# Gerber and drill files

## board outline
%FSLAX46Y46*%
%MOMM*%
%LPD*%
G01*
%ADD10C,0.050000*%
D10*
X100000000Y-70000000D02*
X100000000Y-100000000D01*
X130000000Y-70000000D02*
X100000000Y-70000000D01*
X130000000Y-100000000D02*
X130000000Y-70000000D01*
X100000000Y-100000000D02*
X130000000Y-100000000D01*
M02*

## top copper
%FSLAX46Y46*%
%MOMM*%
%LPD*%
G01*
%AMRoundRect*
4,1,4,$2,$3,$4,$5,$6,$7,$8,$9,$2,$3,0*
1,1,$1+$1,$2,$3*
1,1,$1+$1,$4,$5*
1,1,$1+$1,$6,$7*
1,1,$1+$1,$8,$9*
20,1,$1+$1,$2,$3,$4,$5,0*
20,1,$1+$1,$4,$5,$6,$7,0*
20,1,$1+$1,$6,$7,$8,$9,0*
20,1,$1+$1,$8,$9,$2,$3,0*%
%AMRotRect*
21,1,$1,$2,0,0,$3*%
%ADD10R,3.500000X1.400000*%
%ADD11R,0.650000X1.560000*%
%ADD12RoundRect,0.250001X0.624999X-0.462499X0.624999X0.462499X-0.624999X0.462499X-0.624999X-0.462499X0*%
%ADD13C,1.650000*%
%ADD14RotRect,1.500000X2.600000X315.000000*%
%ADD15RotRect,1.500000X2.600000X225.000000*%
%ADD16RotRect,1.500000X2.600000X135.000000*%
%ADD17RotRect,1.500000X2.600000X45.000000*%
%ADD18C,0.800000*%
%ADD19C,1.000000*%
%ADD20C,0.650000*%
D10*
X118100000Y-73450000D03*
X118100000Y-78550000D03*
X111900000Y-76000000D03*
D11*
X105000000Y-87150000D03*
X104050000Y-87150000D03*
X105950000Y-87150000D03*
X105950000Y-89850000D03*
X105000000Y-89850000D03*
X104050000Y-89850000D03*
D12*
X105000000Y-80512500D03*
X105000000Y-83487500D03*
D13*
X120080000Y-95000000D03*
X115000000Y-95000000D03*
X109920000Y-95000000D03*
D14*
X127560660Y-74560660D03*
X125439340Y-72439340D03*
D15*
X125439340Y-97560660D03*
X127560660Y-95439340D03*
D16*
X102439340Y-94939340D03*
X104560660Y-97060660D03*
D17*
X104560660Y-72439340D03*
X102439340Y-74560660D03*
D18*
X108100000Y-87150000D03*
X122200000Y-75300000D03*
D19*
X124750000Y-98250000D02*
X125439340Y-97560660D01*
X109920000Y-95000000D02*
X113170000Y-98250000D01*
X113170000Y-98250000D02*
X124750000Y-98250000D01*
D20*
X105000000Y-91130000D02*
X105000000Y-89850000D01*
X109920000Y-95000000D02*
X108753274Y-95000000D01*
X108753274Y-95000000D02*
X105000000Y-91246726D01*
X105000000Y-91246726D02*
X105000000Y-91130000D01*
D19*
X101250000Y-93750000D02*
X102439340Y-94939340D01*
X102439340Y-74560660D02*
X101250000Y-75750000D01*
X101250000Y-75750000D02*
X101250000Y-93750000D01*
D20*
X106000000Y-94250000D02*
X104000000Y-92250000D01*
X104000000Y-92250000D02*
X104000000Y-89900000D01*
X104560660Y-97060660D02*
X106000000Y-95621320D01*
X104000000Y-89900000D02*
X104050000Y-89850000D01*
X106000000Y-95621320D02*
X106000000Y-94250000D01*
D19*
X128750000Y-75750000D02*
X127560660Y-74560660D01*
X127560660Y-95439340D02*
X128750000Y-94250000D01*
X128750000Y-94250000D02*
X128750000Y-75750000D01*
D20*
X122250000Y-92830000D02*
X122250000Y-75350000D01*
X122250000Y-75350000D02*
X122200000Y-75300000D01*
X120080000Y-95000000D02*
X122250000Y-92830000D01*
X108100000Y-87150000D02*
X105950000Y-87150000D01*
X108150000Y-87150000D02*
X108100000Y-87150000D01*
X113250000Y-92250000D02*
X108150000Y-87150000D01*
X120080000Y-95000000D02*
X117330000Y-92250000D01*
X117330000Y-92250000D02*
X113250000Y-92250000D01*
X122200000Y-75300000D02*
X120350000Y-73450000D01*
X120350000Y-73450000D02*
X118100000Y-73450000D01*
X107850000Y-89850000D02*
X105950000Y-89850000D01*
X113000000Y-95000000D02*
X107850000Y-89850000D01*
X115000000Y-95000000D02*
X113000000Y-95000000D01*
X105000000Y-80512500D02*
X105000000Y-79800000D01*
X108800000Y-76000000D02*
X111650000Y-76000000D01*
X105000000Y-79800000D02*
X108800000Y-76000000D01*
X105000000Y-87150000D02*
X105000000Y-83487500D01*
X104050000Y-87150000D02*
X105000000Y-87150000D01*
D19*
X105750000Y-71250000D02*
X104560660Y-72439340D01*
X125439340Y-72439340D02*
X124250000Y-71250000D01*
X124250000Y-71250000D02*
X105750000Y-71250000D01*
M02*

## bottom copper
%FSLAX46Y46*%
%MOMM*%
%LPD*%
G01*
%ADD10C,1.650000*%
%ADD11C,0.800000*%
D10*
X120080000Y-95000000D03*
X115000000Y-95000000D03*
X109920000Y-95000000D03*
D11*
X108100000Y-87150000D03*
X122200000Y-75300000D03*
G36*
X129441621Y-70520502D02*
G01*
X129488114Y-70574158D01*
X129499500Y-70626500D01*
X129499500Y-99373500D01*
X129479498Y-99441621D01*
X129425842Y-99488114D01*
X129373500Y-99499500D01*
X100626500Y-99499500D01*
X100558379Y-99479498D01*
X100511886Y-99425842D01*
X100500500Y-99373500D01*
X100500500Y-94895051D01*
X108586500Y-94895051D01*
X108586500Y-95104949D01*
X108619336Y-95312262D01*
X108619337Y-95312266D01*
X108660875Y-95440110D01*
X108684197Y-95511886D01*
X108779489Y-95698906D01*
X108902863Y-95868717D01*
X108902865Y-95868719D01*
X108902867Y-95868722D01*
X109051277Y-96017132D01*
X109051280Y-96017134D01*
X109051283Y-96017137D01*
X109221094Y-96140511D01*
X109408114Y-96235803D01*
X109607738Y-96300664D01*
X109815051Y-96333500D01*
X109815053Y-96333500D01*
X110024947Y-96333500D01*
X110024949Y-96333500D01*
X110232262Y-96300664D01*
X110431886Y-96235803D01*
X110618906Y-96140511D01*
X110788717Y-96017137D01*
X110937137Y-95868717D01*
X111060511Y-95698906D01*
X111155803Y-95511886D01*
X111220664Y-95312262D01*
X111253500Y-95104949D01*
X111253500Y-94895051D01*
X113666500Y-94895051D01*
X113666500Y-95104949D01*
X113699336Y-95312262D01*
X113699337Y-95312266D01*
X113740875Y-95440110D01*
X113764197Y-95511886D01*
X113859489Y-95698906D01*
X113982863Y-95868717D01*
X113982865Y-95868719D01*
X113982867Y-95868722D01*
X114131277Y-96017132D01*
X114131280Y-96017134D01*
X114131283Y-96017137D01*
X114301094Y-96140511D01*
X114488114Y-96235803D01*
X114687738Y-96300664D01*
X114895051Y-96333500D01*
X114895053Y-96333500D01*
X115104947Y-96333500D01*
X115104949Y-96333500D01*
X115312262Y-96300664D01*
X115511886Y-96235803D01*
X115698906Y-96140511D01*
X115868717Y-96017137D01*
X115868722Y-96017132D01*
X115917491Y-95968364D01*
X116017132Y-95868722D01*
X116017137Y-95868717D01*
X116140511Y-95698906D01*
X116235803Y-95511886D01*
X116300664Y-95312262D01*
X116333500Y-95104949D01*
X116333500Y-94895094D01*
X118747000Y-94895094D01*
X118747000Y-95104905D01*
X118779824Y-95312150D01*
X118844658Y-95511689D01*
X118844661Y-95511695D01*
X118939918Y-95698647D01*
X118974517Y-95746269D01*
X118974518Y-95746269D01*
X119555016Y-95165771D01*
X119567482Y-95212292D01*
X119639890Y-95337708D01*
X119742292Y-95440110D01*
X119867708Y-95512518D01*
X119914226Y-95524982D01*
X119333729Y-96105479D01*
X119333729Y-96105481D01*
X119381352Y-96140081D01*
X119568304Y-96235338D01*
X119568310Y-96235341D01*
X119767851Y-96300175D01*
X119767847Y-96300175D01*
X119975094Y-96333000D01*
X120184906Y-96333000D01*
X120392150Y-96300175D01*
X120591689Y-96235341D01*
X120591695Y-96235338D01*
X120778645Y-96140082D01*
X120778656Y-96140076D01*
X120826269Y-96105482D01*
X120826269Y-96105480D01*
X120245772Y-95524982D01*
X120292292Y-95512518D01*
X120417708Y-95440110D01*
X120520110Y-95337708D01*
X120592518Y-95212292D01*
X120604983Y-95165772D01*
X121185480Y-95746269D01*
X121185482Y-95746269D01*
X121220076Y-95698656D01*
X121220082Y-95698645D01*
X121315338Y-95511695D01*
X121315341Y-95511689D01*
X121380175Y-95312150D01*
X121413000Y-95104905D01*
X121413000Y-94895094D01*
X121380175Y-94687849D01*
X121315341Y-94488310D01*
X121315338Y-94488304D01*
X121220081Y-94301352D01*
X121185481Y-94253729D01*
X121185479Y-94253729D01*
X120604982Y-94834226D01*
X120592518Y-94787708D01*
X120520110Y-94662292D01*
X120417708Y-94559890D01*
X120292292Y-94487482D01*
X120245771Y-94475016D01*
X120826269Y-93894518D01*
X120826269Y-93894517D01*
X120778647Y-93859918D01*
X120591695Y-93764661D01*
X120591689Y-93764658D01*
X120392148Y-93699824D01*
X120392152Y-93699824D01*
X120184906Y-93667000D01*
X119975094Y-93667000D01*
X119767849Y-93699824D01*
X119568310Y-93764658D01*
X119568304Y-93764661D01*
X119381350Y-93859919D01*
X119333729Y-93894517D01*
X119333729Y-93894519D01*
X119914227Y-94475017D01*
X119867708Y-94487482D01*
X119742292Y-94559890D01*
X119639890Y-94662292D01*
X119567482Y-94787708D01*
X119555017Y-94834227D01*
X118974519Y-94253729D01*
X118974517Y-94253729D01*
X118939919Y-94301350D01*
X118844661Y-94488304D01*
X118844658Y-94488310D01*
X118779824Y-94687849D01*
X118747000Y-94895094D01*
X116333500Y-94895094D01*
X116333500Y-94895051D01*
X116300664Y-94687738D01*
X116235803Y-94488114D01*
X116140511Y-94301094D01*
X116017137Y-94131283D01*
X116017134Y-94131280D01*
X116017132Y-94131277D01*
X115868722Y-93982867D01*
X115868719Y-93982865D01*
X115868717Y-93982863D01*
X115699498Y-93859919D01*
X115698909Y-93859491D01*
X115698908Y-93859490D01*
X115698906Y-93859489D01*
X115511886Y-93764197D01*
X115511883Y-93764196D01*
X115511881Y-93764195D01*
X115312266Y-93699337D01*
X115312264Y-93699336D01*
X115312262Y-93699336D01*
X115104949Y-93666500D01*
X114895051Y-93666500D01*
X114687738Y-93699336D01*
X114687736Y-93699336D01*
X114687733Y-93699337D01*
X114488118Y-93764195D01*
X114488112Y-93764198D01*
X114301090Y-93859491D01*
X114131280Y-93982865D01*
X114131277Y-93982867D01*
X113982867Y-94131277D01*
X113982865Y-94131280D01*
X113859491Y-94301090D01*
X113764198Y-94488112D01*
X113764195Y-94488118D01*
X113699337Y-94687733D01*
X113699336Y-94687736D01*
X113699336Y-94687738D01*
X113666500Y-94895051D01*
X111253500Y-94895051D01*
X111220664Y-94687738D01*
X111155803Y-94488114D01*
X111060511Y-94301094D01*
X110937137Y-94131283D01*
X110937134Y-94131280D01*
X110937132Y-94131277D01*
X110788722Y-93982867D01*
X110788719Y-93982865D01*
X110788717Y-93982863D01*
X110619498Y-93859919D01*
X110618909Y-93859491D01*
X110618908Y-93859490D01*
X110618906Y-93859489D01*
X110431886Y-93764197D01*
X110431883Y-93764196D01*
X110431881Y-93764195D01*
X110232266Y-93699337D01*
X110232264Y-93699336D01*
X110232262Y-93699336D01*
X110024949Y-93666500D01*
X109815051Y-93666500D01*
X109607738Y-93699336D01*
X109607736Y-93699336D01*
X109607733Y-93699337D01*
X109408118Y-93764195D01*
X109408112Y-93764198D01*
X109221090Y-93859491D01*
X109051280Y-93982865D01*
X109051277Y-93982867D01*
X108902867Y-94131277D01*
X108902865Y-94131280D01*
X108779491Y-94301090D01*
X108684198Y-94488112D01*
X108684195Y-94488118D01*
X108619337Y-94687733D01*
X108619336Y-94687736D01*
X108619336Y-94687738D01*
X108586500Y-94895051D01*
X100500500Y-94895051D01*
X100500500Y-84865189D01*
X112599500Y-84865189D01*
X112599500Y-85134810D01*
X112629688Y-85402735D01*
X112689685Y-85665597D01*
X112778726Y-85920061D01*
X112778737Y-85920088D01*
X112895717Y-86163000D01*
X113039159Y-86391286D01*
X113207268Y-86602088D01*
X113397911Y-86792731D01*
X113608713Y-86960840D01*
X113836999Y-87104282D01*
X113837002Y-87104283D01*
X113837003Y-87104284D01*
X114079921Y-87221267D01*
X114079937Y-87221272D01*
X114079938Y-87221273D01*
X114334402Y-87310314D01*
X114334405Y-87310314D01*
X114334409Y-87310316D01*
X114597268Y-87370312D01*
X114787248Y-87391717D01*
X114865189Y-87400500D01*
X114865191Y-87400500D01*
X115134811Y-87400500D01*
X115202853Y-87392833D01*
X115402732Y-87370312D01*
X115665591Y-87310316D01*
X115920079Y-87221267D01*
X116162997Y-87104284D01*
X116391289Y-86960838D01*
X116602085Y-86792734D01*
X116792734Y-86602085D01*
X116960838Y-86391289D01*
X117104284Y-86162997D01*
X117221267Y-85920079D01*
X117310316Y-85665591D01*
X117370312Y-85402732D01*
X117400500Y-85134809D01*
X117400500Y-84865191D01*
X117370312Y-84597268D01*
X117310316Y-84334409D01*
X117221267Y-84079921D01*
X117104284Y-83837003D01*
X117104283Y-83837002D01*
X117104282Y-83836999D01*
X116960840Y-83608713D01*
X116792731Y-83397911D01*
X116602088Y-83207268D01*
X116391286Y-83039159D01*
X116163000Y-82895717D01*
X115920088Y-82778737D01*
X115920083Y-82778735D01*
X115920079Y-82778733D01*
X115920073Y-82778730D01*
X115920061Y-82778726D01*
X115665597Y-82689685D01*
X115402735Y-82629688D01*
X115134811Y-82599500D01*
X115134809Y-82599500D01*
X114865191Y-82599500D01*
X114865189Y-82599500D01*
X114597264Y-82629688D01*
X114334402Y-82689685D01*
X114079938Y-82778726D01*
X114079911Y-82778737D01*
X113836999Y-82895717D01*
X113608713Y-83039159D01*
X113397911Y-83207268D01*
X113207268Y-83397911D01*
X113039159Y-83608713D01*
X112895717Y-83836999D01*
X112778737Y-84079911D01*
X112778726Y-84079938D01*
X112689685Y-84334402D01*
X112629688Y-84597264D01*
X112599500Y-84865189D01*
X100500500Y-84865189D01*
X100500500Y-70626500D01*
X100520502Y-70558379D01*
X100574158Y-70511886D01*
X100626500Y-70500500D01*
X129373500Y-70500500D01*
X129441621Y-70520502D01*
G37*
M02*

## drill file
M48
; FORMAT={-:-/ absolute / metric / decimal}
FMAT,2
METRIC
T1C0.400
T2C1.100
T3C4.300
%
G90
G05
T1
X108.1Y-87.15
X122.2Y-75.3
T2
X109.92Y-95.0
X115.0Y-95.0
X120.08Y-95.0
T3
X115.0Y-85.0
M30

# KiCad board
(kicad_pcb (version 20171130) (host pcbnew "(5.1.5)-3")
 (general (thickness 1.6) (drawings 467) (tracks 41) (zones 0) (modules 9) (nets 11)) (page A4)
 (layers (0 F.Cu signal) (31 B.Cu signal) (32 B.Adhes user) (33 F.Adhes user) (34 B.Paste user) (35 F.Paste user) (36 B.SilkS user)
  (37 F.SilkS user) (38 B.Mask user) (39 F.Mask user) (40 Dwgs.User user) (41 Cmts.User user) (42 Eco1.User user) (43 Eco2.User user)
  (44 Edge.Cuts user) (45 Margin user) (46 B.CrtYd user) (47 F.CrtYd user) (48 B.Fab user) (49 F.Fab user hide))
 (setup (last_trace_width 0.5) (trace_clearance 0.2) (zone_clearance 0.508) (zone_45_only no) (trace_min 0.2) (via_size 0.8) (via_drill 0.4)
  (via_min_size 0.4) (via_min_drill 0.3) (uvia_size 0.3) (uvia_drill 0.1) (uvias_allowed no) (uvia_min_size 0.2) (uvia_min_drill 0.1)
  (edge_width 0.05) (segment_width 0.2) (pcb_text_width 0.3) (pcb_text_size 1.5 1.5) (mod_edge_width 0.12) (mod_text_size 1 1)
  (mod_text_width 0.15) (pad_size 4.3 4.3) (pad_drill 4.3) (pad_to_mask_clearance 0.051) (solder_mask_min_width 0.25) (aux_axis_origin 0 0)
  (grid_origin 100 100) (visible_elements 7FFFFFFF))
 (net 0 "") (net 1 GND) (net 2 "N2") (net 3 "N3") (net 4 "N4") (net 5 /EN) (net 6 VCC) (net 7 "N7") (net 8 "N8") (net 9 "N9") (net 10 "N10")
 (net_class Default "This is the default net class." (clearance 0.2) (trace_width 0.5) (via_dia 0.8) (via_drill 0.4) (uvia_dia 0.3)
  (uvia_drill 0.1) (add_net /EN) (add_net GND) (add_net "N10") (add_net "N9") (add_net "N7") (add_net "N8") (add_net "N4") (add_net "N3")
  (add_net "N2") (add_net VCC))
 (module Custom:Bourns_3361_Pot (layer F.Cu) (at 115 76 90)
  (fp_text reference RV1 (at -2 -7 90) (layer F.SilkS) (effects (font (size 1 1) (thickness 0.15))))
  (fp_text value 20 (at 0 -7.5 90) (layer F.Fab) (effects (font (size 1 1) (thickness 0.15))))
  (pad 3 smd rect (at 2.55 3.1 90) (size 1.4 3.5) (layers F.Cu F.Paste F.Mask) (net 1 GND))
  (pad 1 smd rect (at -2.55 3.1 90) (size 1.4 3.5) (layers F.Cu F.Paste F.Mask) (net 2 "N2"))
  (pad 2 smd rect (at 0 -3.1 90) (size 1.4 3.5) (layers F.Cu F.Paste F.Mask) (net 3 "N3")))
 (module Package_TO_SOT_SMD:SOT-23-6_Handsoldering (layer F.Cu) (at 105 88.5 90)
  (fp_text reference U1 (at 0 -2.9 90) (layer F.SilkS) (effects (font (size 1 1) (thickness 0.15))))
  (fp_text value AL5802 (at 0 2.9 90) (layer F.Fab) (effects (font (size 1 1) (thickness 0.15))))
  (pad 5 smd rect (at 1.35 0 90) (size 1.56 0.65) (layers F.Cu F.Paste F.Mask) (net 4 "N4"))
  (pad 6 smd rect (at 1.35 -0.95 90) (size 1.56 0.65) (layers F.Cu F.Paste F.Mask) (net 4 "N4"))
  (pad 4 smd rect (at 1.35 0.95 90) (size 1.56 0.65) (layers F.Cu F.Paste F.Mask) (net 1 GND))
  (pad 3 smd rect (at -1.35 0.95 90) (size 1.56 0.65) (layers F.Cu F.Paste F.Mask) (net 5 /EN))
  (pad 2 smd rect (at -1.35 0 90) (size 1.56 0.65) (layers F.Cu F.Paste F.Mask) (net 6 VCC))
  (pad 1 smd rect (at -1.35 -0.95 90) (size 1.56 0.65) (layers F.Cu F.Paste F.Mask) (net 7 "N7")))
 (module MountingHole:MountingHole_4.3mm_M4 (layer F.Cu) (at 115 85)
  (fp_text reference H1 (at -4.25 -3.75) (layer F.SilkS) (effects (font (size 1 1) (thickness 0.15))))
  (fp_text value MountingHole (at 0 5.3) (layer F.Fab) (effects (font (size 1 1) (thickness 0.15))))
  (pad 1 np_thru_hole circle (at 0 0) (size 4.3 4.3) (drill 4.3) (layers *.Cu *.Mask)))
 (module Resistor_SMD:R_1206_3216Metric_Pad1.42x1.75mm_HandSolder (layer F.Cu) (at 105 82 90)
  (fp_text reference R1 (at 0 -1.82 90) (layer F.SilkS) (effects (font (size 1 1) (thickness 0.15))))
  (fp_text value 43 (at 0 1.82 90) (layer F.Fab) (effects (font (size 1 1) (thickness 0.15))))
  (pad 2 smd roundrect (at 1.4875 0 90) (size 1.425 1.75) (layers F.Cu F.Paste F.Mask) (roundrect_rratio 0.175439) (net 3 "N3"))
  (pad 1 smd roundrect (at -1.4875 0 90) (size 1.425 1.75) (layers F.Cu F.Paste F.Mask) (roundrect_rratio 0.175439) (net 4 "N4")))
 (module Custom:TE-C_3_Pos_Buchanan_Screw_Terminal (layer F.Cu) (at 115 95)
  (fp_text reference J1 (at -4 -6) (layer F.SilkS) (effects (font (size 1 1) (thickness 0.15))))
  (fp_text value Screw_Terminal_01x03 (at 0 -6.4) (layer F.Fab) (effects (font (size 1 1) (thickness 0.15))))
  (pad 3 thru_hole circle (at 5.08 0) (size 1.65 1.65) (drill 1.1) (layers *.Cu *.Mask) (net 1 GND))
  (pad 2 thru_hole circle (at 0 0) (size 1.65 1.65) (drill 1.1) (layers *.Cu *.Mask) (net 5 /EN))
  (pad 1 thru_hole circle (at -5.08 0) (size 1.65 1.65) (drill 1.1) (layers *.Cu *.Mask) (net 6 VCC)))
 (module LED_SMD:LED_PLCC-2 (layer F.Cu) (at 126.5 73.5 315)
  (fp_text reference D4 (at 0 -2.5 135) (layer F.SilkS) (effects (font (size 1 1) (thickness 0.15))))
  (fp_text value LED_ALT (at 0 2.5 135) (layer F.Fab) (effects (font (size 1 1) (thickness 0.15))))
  (pad 2 smd rect (at 1.5 0 315) (size 1.5 2.6) (layers F.Cu F.Paste F.Mask) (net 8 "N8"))
  (pad 1 smd rect (at -1.5 0 315) (size 1.5 2.6) (layers F.Cu F.Paste F.Mask) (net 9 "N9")))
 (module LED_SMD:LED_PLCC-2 (layer F.Cu) (at 126.5 96.5 225)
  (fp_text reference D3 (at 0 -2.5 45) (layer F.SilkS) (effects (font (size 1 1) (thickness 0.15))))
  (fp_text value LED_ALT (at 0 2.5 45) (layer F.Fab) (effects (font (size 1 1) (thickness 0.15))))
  (pad 2 smd rect (at 1.5 0 225) (size 1.5 2.6) (layers F.Cu F.Paste F.Mask) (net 6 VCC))
  (pad 1 smd rect (at -1.5 0 225) (size 1.5 2.6) (layers F.Cu F.Paste F.Mask) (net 8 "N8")))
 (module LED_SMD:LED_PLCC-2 (layer F.Cu) (at 103.5 96 135)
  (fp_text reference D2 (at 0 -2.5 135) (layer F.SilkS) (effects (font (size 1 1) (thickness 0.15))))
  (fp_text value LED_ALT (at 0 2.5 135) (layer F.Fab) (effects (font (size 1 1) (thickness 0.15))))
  (pad 2 smd rect (at 1.5 0 135) (size 1.5 2.6) (layers F.Cu F.Paste F.Mask) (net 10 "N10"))
  (pad 1 smd rect (at -1.5 0 135) (size 1.5 2.6) (layers F.Cu F.Paste F.Mask) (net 7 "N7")))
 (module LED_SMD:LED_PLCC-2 (layer F.Cu) (at 103.5 73.5 45)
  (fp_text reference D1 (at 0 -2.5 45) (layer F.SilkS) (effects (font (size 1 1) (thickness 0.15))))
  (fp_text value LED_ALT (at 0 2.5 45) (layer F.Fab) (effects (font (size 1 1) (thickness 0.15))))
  (pad 2 smd rect (at 1.5 0 45) (size 1.5 2.6) (layers F.Cu F.Paste F.Mask) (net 9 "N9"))
  (pad 1 smd rect (at -1.5 0 45) (size 1.5 2.6) (layers F.Cu F.Paste F.Mask) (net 10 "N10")))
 (gr_line (start 100 70) (end 100 100) (layer Edge.Cuts) (width 0.05))
 (gr_line (start 130 70) (end 100 70) (layer Edge.Cuts) (width 0.05))
 (gr_line (start 130 100) (end 130 70) (layer Edge.Cuts) (width 0.05))
 (gr_line (start 100 100) (end 130 100) (layer Edge.Cuts) (width 0.05))
 (segment (start 124.75 98.25) (end 125.43934 97.56066) (width 1) (layer F.Cu) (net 6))
 (segment (start 109.92 95) (end 113.17 98.25) (width 1) (layer F.Cu) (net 6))
 (segment (start 113.17 98.25) (end 124.75 98.25) (width 1) (layer F.Cu) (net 6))
 (segment (start 105 91.13) (end 105 89.85) (width 0.65) (layer F.Cu) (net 6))
 (segment (start 109.92 95) (end 108.753274 95) (width 0.65) (layer F.Cu) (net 6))
 (segment (start 108.753274 95) (end 105 91.246726) (width 0.65) (layer F.Cu) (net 6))
 (segment (start 105 91.246726) (end 105 91.13) (width 0.65) (layer F.Cu) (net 6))
 (segment (start 101.25 93.75) (end 102.43934 94.93934) (width 1) (layer F.Cu) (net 10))
 (segment (start 102.43934 74.56066) (end 101.25 75.75) (width 1) (layer F.Cu) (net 10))
 (segment (start 101.25 75.75) (end 101.25 93.75) (width 1) (layer F.Cu) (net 10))
 (segment (start 106 94.25) (end 104 92.25) (width 0.65) (layer F.Cu) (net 7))
 (segment (start 104 92.25) (end 104 89.9) (width 0.65) (layer F.Cu) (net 7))
 (segment (start 104.56066 97.06066) (end 106 95.62132) (width 0.65) (layer F.Cu) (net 7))
 (segment (start 104 89.9) (end 104.05 89.85) (width 0.65) (layer F.Cu) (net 7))
 (segment (start 106 95.62132) (end 106 94.25) (width 0.65) (layer F.Cu) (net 7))
 (segment (start 128.75 75.75) (end 127.56066 74.56066) (width 1) (layer F.Cu) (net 8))
 (segment (start 127.56066 95.43934) (end 128.75 94.25) (width 1) (layer F.Cu) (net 8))
 (segment (start 128.75 94.25) (end 128.75 75.75) (width 1) (layer F.Cu) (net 8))
 (segment (start 122.25 92.83) (end 122.25 75.35) (width 0.65) (layer F.Cu) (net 1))
 (segment (start 122.25 75.35) (end 122.2 75.3) (width 0.65) (layer F.Cu) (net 1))
 (segment (start 120.08 95) (end 122.25 92.83) (width 0.65) (layer F.Cu) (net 1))
 (segment (start 108.1 87.15) (end 105.95 87.15) (width 0.65) (layer F.Cu) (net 1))
 (via (at 108.1 87.15) (size 0.8) (drill 0.4) (layers F.Cu B.Cu) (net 1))
 (via (at 122.2 75.3) (size 0.8) (drill 0.4) (layers F.Cu B.Cu) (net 1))
 (segment (start 108.15 87.15) (end 108.1 87.15) (width 0.65) (layer F.Cu) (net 1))
 (segment (start 113.25 92.25) (end 108.15 87.15) (width 0.65) (layer F.Cu) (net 1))
 (segment (start 120.08 95) (end 117.33 92.25) (width 0.65) (layer F.Cu) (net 1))
 (segment (start 117.33 92.25) (end 113.25 92.25) (width 0.65) (layer F.Cu) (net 1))
 (segment (start 122.2 75.3) (end 120.35 73.45) (width 0.65) (layer F.Cu) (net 1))
 (segment (start 120.35 73.45) (end 118.1 73.45) (width 0.65) (layer F.Cu) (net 1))
 (segment (start 107.85 89.85) (end 105.95 89.85) (width 0.65) (layer F.Cu) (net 5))
 (segment (start 113 95) (end 107.85 89.85) (width 0.65) (layer F.Cu) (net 5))
 (segment (start 115 95) (end 113 95) (width 0.65) (layer F.Cu) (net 5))
 (segment (start 105 80.5125) (end 105 79.8) (width 0.65) (layer F.Cu) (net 3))
 (segment (start 108.8 76) (end 111.65 76) (width 0.65) (layer F.Cu) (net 3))
 (segment (start 105 79.8) (end 108.8 76) (width 0.65) (layer F.Cu) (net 3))
 (segment (start 105 87.15) (end 105 83.4875) (width 0.65) (layer F.Cu) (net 4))
 (segment (start 104.05 87.15) (end 105 87.15) (width 0.65) (layer F.Cu) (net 4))
 (segment (start 105.75 71.25) (end 104.56066 72.43934) (width 1) (layer F.Cu) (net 9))
 (segment (start 125.43934 72.43934) (end 124.25 71.25) (width 1) (layer F.Cu) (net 9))
 (segment (start 124.25 71.25) (end 105.75 71.25) (width 1) (layer F.Cu) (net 9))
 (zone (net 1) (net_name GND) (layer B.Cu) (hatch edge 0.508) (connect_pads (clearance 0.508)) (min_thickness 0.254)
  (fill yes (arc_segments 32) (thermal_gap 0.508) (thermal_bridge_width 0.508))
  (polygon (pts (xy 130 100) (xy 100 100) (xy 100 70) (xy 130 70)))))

